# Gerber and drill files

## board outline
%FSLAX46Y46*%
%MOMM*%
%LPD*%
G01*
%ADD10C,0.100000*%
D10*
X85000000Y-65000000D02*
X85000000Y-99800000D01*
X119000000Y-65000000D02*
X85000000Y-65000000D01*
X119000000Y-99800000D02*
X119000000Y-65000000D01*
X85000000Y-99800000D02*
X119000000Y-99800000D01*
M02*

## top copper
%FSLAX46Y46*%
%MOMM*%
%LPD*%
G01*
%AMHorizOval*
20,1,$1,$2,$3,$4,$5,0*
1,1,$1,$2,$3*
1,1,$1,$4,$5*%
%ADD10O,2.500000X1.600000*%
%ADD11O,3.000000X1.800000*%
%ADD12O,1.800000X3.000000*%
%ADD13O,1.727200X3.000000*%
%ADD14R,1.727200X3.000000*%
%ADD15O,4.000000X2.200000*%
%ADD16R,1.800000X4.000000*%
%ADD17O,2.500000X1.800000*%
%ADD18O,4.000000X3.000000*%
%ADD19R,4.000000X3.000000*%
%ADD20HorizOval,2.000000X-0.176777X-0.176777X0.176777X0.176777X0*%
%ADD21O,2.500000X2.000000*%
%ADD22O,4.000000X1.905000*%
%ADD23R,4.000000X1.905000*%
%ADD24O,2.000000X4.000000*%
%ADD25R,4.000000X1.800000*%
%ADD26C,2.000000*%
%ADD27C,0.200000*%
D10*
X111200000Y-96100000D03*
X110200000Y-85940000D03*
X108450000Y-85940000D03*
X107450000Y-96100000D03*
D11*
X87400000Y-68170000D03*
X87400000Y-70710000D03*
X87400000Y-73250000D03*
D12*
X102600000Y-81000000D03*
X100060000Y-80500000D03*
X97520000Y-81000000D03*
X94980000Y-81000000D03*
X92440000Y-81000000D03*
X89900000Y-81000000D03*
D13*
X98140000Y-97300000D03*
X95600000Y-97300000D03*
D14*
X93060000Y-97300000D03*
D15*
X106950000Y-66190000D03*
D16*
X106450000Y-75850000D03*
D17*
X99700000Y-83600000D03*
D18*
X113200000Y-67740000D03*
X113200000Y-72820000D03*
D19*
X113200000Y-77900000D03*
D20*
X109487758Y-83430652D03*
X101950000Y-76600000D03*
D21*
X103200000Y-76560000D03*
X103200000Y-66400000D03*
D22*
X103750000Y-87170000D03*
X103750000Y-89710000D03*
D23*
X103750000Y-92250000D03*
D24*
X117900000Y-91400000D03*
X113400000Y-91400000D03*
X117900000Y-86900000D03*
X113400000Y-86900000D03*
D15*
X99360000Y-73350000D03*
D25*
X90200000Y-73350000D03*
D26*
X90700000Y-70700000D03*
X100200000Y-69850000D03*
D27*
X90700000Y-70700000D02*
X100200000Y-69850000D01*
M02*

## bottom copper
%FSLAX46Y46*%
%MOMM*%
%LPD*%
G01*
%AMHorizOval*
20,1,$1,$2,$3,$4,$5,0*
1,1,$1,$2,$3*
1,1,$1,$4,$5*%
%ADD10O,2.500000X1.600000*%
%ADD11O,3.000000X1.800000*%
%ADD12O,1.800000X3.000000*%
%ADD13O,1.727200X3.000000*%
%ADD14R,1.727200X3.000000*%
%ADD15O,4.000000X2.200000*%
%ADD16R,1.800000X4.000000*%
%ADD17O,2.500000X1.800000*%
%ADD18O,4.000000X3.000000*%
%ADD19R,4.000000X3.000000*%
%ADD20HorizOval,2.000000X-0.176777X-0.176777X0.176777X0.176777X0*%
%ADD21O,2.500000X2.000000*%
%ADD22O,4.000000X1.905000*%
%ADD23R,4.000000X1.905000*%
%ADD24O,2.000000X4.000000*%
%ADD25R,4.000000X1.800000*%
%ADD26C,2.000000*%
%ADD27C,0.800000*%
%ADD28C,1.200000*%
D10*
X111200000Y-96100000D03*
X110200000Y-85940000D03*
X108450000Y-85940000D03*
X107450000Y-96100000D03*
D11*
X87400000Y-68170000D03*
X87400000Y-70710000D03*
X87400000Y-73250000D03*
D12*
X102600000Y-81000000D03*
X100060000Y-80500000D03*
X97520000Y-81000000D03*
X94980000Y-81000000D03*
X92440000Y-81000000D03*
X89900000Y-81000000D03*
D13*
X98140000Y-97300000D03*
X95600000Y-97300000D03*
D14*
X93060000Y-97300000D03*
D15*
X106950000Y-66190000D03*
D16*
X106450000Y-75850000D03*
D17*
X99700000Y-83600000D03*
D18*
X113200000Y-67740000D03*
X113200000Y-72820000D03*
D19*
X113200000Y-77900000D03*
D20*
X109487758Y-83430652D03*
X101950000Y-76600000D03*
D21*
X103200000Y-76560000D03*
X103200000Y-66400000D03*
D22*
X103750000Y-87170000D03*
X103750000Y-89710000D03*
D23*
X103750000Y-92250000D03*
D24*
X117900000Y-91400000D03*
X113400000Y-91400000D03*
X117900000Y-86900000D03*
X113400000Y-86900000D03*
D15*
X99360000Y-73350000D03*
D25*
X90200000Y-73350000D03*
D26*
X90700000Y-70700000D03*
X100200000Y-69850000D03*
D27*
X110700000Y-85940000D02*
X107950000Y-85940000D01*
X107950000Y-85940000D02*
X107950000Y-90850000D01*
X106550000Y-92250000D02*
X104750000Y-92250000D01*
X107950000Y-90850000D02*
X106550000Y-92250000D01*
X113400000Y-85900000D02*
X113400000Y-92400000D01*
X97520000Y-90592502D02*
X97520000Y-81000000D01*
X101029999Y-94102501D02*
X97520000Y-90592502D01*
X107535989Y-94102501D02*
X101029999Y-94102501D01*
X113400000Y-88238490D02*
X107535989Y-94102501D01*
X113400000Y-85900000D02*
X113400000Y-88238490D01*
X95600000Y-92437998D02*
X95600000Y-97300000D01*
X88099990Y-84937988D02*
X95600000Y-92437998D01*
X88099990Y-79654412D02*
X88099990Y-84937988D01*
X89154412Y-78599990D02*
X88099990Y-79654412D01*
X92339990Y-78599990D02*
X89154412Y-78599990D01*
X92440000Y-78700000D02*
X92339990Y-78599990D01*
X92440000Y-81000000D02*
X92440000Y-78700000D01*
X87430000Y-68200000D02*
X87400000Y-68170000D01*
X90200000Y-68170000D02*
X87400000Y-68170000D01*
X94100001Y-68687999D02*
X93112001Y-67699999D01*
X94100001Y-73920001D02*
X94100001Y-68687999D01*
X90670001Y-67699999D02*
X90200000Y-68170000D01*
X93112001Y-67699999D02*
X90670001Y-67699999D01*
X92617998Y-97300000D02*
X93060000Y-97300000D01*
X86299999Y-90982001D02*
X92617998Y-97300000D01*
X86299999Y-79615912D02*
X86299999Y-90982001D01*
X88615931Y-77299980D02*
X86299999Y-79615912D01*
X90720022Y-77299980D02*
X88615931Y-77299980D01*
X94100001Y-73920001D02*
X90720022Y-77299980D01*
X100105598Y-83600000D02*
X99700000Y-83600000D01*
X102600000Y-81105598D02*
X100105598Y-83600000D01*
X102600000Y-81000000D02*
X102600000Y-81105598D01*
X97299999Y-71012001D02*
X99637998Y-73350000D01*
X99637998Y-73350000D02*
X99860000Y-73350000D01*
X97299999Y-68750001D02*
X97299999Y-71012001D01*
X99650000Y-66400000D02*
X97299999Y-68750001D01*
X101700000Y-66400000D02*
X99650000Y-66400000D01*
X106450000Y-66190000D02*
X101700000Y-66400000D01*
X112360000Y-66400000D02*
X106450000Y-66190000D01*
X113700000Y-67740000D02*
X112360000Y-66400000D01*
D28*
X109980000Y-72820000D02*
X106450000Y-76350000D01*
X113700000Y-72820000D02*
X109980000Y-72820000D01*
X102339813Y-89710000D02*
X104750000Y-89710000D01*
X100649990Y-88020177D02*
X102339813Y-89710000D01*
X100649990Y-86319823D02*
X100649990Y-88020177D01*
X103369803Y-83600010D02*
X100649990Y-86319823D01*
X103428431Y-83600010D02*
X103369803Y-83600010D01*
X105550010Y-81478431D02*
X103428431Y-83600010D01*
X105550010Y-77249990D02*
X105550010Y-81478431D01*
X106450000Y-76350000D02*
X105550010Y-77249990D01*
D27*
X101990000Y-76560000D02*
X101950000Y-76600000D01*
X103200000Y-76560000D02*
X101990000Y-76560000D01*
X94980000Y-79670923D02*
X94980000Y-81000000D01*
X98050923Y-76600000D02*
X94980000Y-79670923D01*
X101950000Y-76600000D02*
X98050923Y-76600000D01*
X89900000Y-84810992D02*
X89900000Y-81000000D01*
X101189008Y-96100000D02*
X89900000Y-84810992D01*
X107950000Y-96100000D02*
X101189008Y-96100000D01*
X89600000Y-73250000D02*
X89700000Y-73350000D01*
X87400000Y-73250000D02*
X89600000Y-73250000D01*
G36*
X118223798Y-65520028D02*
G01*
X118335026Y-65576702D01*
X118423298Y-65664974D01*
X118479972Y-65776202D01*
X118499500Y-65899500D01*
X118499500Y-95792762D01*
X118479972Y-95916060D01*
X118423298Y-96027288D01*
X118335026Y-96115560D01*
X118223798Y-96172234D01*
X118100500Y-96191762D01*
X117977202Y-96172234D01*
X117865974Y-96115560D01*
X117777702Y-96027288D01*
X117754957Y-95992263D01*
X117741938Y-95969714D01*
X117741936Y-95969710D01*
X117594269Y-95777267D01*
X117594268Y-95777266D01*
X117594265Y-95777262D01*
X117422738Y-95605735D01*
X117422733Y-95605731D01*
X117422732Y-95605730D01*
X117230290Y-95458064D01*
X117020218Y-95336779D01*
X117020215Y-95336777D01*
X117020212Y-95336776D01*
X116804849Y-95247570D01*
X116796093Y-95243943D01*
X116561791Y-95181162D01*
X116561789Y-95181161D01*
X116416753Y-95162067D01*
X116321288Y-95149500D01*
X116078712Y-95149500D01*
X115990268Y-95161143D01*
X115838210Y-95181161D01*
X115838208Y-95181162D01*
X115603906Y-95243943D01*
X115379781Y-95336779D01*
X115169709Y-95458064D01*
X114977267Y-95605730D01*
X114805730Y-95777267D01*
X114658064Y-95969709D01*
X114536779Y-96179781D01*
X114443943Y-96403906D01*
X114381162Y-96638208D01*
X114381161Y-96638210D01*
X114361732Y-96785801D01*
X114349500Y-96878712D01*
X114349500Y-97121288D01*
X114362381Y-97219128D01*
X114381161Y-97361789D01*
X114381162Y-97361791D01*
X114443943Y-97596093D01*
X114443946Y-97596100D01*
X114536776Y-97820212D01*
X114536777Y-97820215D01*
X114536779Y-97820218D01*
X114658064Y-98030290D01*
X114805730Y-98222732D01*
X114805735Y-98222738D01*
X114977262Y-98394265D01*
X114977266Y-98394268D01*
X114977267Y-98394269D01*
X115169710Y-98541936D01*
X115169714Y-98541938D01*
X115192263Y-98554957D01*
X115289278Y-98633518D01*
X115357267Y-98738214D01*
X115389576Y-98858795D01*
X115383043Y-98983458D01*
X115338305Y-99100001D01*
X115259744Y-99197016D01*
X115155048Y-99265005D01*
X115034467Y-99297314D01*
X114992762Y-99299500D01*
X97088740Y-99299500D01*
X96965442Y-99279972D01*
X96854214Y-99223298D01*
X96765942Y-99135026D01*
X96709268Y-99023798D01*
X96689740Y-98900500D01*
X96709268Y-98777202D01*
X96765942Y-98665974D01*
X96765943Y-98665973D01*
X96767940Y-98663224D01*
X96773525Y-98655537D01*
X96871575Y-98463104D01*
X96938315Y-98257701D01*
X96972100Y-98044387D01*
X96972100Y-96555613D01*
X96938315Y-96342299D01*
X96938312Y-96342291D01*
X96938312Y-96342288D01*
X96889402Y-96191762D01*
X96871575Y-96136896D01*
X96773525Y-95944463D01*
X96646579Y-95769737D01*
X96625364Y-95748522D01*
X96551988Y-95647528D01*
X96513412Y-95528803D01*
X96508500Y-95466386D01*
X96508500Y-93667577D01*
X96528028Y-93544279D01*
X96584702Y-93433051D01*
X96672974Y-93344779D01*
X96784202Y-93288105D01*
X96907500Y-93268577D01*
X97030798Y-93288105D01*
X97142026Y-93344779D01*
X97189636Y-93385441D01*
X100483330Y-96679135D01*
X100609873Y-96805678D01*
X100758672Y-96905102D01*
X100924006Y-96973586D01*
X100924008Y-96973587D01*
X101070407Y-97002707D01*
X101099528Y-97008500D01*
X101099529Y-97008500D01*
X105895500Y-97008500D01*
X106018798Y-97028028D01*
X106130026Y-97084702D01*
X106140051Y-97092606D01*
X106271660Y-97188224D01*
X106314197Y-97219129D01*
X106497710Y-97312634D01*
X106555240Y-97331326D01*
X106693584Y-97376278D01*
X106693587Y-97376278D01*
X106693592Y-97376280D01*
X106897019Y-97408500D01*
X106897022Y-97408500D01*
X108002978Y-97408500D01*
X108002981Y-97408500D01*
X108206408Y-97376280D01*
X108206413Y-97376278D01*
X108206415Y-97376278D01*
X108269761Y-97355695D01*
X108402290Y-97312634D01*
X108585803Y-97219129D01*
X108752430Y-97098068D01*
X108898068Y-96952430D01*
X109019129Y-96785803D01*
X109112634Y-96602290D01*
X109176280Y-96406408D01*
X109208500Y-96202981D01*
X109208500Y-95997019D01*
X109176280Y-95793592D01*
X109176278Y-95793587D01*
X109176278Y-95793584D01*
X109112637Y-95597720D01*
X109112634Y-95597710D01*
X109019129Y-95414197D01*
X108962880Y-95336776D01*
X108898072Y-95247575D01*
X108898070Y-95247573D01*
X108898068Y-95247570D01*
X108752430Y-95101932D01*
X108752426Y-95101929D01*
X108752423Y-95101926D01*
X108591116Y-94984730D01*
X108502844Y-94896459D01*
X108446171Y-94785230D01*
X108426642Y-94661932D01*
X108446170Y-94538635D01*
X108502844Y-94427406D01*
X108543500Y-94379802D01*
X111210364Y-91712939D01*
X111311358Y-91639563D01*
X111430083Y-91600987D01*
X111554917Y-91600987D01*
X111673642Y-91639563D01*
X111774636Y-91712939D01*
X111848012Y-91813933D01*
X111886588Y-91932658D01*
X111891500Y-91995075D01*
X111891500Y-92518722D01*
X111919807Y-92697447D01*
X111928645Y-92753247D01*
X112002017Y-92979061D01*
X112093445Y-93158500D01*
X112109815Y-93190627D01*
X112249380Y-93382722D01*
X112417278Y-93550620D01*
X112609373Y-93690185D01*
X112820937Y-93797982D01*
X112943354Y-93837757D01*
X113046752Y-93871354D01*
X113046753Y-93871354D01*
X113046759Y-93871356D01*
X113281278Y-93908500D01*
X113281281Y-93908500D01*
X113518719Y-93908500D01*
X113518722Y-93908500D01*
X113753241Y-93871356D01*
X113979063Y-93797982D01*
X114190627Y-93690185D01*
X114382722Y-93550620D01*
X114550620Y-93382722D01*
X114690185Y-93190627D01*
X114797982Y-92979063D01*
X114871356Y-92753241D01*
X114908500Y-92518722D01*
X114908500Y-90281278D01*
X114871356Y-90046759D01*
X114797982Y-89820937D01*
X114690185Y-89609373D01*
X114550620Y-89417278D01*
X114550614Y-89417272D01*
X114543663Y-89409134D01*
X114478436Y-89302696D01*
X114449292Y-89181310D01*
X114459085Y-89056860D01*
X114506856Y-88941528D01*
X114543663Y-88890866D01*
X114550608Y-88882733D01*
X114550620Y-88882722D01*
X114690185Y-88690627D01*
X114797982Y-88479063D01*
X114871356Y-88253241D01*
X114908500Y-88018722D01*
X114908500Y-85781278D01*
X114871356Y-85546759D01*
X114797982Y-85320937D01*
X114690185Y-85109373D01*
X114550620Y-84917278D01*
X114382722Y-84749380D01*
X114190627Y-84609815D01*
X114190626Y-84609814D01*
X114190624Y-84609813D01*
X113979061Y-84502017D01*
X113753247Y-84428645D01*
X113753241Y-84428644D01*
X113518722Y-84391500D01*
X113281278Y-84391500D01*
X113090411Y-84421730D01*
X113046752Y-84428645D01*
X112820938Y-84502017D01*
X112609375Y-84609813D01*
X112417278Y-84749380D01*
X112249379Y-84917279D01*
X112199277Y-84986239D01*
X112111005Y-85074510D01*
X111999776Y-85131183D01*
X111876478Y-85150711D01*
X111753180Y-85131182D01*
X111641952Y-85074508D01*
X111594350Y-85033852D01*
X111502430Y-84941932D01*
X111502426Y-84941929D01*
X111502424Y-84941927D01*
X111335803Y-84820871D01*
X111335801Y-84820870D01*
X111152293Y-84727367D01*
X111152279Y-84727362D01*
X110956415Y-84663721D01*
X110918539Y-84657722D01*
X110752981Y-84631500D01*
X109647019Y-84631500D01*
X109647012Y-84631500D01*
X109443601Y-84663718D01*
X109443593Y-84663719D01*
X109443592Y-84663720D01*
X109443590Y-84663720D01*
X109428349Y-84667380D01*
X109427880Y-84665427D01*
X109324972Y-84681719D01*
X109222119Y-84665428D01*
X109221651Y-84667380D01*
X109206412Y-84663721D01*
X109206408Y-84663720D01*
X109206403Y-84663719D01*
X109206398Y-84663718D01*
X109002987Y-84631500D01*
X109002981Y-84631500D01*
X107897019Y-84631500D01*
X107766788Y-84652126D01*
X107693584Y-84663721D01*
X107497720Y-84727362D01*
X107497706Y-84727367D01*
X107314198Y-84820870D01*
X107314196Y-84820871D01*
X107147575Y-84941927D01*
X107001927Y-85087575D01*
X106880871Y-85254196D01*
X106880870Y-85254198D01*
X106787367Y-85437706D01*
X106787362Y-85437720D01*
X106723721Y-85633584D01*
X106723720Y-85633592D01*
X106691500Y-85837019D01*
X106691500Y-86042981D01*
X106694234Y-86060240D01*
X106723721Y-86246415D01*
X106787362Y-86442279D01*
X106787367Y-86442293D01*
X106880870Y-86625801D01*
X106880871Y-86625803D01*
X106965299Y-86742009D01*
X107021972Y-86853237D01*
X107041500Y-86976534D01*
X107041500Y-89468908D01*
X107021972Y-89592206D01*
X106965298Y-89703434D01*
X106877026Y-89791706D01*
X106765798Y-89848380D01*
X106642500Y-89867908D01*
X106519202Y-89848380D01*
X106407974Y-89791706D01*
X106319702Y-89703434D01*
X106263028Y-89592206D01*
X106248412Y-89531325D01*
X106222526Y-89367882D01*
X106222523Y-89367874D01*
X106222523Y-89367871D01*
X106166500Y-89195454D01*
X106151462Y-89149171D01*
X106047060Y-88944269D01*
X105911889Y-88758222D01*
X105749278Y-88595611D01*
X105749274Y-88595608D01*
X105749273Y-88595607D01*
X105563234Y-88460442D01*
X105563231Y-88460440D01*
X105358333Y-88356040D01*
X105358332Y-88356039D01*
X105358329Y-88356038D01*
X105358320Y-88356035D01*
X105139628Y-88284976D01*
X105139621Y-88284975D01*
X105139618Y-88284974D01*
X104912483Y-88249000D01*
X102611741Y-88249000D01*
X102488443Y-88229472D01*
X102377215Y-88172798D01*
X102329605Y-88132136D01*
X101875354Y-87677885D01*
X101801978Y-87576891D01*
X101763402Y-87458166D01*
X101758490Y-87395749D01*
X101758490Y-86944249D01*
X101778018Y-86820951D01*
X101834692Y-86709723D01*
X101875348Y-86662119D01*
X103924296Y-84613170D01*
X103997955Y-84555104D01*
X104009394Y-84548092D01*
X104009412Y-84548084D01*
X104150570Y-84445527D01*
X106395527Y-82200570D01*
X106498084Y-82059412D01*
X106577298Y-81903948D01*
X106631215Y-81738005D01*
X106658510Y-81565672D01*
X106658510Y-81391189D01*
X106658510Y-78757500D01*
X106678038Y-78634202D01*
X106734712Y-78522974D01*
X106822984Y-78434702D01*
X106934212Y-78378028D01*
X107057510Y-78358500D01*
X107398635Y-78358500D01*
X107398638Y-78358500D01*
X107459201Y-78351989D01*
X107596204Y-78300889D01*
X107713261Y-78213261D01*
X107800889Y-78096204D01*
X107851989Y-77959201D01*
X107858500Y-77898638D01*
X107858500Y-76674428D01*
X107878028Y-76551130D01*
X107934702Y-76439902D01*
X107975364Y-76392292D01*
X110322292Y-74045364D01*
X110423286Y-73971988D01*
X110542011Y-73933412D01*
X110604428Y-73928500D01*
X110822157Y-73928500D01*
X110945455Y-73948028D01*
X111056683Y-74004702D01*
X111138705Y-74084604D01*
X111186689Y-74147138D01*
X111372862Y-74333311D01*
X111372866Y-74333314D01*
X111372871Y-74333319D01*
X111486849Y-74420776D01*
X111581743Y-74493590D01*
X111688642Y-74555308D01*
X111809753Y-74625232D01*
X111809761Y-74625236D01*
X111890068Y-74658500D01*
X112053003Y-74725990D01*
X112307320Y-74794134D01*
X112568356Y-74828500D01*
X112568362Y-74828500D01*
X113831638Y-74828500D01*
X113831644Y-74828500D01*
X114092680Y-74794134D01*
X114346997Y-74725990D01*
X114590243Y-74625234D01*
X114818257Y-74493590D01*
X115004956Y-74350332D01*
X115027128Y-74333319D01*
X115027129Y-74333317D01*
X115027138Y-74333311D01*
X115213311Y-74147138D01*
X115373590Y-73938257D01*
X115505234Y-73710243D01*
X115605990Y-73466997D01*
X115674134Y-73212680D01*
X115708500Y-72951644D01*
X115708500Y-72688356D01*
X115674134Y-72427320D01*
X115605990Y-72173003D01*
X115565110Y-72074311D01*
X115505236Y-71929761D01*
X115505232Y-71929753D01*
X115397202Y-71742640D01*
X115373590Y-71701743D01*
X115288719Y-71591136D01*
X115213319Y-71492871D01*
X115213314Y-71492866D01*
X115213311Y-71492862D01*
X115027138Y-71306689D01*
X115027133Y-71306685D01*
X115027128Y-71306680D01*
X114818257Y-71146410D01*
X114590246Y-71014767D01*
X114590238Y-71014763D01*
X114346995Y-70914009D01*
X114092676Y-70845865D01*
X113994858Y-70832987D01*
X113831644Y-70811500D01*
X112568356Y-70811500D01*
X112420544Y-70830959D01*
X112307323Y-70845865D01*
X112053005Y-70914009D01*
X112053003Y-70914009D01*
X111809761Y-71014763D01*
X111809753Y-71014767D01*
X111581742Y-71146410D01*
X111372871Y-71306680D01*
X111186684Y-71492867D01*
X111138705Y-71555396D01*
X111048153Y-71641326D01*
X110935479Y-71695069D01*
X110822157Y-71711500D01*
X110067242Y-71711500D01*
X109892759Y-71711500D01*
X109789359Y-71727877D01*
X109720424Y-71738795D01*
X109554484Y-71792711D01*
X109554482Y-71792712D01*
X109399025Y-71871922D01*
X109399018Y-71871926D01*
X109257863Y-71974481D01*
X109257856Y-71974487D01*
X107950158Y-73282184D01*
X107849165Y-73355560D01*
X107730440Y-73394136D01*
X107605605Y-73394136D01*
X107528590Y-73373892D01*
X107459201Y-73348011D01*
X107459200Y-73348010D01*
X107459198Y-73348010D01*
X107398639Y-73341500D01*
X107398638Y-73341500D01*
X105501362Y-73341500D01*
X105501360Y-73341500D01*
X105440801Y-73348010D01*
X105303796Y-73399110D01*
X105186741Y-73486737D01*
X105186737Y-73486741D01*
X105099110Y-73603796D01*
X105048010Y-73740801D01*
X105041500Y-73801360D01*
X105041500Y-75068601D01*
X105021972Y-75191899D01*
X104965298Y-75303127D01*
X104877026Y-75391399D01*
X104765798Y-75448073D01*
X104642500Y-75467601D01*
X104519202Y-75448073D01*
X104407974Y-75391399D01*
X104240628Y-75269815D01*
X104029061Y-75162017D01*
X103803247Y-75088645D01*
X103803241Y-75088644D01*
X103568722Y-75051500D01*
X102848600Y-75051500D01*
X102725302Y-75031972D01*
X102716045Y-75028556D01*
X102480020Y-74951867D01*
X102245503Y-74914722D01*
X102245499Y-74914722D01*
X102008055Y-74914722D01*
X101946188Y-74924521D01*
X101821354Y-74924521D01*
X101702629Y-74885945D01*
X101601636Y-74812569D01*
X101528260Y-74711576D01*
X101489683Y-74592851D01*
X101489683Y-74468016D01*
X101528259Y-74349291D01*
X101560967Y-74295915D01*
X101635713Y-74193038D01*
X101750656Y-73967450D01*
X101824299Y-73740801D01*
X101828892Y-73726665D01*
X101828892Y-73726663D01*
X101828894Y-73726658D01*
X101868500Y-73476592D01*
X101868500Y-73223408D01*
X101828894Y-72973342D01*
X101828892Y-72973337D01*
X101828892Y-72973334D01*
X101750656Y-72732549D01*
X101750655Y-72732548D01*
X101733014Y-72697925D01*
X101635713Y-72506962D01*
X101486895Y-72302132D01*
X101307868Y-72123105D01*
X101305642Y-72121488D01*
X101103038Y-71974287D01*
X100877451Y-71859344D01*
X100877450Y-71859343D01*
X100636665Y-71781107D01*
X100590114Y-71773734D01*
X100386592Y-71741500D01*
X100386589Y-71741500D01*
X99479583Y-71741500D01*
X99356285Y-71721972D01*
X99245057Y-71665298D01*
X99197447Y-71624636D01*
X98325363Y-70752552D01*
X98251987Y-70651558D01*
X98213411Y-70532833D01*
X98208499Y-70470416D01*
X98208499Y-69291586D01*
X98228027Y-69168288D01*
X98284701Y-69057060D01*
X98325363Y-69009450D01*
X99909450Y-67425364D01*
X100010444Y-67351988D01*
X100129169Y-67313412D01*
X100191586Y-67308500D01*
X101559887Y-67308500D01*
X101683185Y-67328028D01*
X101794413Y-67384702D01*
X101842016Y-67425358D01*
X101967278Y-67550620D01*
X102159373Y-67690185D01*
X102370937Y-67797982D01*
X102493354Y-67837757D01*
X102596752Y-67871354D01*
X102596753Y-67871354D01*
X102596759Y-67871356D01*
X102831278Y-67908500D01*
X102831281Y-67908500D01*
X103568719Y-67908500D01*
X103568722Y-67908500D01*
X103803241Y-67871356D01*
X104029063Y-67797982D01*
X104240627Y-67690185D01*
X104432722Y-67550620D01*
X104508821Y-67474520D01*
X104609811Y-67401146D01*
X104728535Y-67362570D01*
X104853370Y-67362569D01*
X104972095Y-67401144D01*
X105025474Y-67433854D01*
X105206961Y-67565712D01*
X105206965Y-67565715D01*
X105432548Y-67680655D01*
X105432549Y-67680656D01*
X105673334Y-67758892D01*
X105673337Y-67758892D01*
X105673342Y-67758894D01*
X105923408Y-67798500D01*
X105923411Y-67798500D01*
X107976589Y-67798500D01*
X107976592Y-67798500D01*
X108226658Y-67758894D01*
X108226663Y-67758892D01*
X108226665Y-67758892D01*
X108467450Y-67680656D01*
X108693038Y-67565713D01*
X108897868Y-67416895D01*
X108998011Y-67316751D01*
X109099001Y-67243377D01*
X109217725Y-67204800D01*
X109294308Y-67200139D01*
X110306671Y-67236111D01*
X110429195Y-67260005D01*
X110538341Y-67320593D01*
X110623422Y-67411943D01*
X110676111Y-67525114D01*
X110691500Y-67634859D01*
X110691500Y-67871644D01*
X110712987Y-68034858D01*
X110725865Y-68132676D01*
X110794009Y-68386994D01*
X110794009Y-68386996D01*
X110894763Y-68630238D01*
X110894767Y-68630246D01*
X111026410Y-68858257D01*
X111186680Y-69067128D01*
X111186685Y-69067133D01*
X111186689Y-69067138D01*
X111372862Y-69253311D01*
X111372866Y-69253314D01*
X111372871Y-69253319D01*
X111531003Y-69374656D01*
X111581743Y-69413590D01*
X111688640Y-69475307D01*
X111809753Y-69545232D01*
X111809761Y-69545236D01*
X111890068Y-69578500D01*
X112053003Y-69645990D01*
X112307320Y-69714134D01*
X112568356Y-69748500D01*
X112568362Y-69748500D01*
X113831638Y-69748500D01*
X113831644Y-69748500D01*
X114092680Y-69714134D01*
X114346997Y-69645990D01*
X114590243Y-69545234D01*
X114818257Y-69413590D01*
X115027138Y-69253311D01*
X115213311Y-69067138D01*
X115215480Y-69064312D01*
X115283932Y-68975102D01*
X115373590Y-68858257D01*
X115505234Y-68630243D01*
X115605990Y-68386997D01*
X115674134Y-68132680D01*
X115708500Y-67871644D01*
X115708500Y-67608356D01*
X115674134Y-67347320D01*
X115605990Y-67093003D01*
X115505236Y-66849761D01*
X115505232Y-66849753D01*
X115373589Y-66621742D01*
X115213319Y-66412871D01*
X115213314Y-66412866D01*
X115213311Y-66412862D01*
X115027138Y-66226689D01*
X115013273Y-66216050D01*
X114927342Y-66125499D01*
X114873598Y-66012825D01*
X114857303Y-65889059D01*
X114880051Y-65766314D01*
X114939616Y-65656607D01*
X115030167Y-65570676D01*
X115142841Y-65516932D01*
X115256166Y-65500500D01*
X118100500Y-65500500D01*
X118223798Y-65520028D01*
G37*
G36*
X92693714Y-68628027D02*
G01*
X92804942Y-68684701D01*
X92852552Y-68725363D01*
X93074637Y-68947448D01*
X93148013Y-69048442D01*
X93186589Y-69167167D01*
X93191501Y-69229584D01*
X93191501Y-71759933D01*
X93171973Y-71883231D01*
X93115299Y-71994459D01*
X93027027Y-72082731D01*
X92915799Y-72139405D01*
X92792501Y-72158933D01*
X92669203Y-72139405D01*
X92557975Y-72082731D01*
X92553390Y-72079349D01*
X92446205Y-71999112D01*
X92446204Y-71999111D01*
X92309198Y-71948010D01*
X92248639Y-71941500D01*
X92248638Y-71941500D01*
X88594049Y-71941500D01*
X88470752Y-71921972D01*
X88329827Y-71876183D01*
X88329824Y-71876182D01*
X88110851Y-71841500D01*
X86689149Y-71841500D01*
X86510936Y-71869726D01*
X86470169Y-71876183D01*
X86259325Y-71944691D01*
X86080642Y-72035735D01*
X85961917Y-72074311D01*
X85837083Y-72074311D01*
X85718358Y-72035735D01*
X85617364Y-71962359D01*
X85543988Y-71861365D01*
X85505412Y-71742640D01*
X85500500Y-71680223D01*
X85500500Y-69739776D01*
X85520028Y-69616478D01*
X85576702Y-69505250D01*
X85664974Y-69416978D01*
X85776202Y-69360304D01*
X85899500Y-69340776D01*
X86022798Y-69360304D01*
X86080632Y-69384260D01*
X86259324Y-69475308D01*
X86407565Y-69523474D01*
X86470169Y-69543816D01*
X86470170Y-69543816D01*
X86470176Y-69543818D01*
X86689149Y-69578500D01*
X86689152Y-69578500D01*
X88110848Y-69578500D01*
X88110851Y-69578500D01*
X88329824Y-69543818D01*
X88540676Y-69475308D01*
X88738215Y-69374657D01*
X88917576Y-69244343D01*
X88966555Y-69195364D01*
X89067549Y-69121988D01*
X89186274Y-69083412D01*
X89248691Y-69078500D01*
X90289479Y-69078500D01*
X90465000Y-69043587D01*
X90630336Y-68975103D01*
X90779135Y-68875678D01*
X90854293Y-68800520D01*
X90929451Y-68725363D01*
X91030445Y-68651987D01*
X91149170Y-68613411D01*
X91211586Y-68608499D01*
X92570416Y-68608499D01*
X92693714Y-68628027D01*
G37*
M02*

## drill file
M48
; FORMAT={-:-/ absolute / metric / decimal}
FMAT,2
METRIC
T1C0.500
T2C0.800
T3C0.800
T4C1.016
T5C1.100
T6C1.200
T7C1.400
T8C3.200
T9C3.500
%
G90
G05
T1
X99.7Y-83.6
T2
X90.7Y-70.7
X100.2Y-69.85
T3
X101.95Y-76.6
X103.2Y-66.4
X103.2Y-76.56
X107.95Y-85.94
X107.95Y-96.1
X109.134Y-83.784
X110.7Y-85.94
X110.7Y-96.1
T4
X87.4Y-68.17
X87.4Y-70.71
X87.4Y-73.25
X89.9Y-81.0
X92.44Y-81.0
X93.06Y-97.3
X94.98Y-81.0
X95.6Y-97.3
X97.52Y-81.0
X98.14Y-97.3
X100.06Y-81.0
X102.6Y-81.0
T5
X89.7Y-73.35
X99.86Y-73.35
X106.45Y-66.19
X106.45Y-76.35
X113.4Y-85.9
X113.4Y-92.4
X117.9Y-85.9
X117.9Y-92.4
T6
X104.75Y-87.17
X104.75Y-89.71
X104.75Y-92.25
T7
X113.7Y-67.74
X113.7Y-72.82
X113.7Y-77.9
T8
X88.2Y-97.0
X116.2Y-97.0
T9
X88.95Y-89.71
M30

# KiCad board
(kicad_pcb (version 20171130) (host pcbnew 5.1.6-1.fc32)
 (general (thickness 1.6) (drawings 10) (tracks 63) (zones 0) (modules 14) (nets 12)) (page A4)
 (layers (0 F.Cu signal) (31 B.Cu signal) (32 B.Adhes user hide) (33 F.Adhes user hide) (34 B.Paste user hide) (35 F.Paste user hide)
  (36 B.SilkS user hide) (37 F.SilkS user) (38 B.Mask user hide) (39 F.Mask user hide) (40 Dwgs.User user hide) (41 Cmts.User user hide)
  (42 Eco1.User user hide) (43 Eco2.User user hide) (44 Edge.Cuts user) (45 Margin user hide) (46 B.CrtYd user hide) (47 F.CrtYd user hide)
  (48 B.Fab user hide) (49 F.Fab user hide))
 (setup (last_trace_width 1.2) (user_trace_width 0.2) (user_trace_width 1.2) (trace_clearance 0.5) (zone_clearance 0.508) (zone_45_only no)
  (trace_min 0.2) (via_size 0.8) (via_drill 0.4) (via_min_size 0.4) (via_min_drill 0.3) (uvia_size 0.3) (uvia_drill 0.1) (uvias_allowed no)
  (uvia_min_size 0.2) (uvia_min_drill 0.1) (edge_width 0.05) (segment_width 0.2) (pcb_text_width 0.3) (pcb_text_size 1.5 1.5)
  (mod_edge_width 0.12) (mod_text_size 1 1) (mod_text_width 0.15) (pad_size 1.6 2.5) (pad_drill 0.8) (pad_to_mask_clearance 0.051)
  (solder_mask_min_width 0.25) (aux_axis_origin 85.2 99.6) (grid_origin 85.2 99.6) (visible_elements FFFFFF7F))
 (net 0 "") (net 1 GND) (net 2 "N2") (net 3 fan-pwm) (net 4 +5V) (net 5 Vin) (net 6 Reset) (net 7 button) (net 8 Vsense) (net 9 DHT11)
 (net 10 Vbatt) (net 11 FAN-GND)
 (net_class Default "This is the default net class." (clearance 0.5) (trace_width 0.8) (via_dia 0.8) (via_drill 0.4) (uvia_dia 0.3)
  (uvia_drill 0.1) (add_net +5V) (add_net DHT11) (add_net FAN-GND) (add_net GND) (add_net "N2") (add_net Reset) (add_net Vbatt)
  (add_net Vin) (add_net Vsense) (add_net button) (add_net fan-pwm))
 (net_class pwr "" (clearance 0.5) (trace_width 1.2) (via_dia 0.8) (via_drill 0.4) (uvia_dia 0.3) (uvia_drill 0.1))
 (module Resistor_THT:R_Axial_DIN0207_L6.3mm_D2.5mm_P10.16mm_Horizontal (layer F.Cu) (at 110.7 85.94 270)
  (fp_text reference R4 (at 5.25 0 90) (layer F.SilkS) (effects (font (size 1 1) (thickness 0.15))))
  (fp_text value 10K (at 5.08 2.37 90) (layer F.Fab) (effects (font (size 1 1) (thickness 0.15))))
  (pad 2 thru_hole oval (at 10.16 0 270) (size 1.6 2.5) (drill 0.8 (offset 0 -0.5)) (layers *.Cu *.Mask) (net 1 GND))
  (pad 1 thru_hole oval (at 0 0 270) (size 1.6 2.5) (drill 0.8 (offset 0 0.5)) (layers *.Cu *.Mask) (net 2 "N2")))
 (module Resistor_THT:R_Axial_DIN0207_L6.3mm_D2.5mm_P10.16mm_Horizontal (layer F.Cu) (at 107.95 96.1 90)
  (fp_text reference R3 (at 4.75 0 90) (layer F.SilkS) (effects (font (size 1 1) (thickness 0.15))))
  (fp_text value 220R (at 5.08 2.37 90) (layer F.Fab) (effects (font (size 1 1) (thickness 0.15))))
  (pad 2 thru_hole oval (at 10.16 0 90) (size 1.6 2.5) (drill 0.8 (offset 0 0.5)) (layers *.Cu *.Mask) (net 2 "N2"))
  (pad 1 thru_hole oval (at 0 0 90) (size 1.6 2.5) (drill 0.8 (offset 0 -0.5)) (layers *.Cu *.Mask) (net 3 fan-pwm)))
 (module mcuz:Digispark (layer F.Cu) (at 96.25 81)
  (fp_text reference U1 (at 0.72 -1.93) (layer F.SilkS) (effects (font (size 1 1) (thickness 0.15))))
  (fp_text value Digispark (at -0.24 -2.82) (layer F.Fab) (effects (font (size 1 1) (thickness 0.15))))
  (pad 9 thru_hole oval (at -8.85 -12.83) (size 3 1.8) (drill 1.016) (layers *.Cu *.Mask) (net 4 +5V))
  (pad 8 thru_hole oval (at -8.85 -10.29) (size 3 1.8) (drill 1.016) (layers *.Cu *.Mask) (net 1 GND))
  (pad 7 thru_hole oval (at -8.85 -7.75) (size 3 1.8) (drill 1.016) (layers *.Cu *.Mask) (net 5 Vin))
  (pad 6 thru_hole oval (at 6.35 0) (size 1.8 3) (drill 1.016) (layers *.Cu *.Mask) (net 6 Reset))
  (pad 5 thru_hole oval (at 3.81 0) (size 1.8 3) (drill 1.016 (offset 0 -0.5)) (layers *.Cu *.Mask))
  (pad 4 thru_hole oval (at 1.27 0) (size 1.8 3) (drill 1.016) (layers *.Cu *.Mask) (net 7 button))
  (pad 3 thru_hole oval (at -1.27 0) (size 1.8 3) (drill 1.016) (layers *.Cu *.Mask) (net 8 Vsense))
  (pad 2 thru_hole oval (at -3.81 0) (size 1.8 3) (drill 1.016) (layers *.Cu *.Mask) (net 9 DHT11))
  (pad 1 thru_hole oval (at -6.35 0) (size 1.8 3) (drill 1.016) (layers *.Cu *.Mask) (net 3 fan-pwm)))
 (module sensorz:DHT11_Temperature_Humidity (layer F.Cu) (at 95.6 97.3)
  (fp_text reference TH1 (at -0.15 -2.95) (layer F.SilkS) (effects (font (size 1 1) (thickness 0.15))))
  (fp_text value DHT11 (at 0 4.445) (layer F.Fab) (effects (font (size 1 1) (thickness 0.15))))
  (pad 3 thru_hole oval (at 2.54 0 90) (size 3 1.7272) (drill 1.016) (layers *.Cu *.Mask) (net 1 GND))
  (pad 2 thru_hole oval (at 0 0 90) (size 3 1.7272) (drill 1.016) (layers *.Cu *.Mask) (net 9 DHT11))
  (pad 1 thru_hole rect (at -2.54 0 90) (size 3 1.7272) (drill 1.016) (layers *.Cu *.Mask) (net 4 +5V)))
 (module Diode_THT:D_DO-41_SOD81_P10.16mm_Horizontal (layer F.Cu) (at 106.45 76.35 90)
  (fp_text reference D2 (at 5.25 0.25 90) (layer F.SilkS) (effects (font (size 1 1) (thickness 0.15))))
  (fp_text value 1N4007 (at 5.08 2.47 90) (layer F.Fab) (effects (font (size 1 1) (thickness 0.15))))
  (pad 2 thru_hole oval (at 10.16 0 180) (size 4 2.2) (drill 1.1 (offset -0.5 0)) (layers *.Cu *.Mask) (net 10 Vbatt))
  (pad 1 thru_hole rect (at 0 0 90) (size 4 1.8) (drill 1.1 (offset 0.5 0)) (layers *.Cu *.Mask) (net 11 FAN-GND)))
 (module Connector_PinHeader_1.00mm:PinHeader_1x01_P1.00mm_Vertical (layer F.Cu) (at 99.7 83.6)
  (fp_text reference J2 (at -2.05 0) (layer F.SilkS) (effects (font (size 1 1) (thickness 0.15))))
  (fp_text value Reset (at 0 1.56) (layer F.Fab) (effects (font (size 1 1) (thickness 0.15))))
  (pad 1 thru_hole oval (at 0 0) (size 2.5 1.8) (drill 0.5) (layers *.Cu *.Mask) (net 6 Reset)))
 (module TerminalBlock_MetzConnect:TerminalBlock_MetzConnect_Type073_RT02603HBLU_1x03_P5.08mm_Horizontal (layer F.Cu) (at 113.7 77.9 90)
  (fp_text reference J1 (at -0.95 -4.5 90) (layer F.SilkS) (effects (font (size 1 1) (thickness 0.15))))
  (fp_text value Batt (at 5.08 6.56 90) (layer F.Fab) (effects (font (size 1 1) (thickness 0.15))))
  (pad 3 thru_hole oval (at 10.16 0 90) (size 3 4) (drill 1.4 (offset 0 -0.5)) (layers *.Cu *.Mask) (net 10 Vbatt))
  (pad 2 thru_hole oval (at 5.08 0 90) (size 3 4) (drill 1.4 (offset 0 -0.5)) (layers *.Cu *.Mask) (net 11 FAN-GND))
  (pad 1 thru_hole rect (at 0 0 90) (size 3 4) (drill 1.4 (offset 0 -0.5)) (layers *.Cu *.Mask) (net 1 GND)))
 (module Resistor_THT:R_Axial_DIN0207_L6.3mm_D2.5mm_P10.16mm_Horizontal (layer F.Cu) (at 101.95 76.6 315)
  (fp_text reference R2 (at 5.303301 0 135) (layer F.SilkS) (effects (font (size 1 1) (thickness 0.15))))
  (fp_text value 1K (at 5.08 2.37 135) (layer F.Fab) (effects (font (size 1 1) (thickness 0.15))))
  (pad 2 thru_hole oval (at 10.16 0 315) (size 2 2.5) (drill 0.8 (offset 0 -0.5)) (layers *.Cu *.Mask) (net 1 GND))
  (pad 1 thru_hole oval (at 0 0 315) (size 2 2.5) (drill 0.8) (layers *.Cu *.Mask) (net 8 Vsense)))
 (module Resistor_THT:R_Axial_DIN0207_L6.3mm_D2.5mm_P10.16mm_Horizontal (layer F.Cu) (at 103.2 66.4 270)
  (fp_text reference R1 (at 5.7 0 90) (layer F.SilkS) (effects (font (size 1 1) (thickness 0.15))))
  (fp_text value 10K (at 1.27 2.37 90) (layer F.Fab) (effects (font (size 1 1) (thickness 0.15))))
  (pad 2 thru_hole oval (at 10.16 0 270) (size 2 2.5) (drill 0.8) (layers *.Cu *.Mask) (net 8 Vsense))
  (pad 1 thru_hole oval (at 0 0 270) (size 2 2.5) (drill 0.8) (layers *.Cu *.Mask) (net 10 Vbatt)))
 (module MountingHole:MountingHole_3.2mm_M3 (layer F.Cu) (at 116.2 97)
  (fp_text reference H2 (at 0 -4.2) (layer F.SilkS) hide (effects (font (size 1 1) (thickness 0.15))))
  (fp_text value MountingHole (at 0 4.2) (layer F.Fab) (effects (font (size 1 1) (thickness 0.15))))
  (pad 1 np_thru_hole circle (at 0 0) (size 3.2 3.2) (drill 3.2) (layers *.Cu *.Mask)))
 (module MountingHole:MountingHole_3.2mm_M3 (layer F.Cu) (at 88.2 97)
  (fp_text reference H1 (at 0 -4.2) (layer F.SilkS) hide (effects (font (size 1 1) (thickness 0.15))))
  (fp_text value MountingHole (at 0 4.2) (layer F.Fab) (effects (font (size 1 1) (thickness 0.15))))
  (pad 1 np_thru_hole circle (at 0 0) (size 3.2 3.2) (drill 3.2) (layers *.Cu *.Mask)))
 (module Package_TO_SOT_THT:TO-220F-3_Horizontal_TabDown (layer F.Cu) (at 104.75 92.25 90)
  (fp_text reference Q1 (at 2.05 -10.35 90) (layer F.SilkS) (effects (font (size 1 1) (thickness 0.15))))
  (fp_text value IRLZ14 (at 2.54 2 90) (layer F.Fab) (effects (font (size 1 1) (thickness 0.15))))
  (pad 3 thru_hole oval (at 5.08 0 90) (size 1.905 4) (drill 1.2 (offset 0 -1)) (layers *.Cu *.Mask) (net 1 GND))
  (pad 2 thru_hole oval (at 2.54 0 90) (size 1.905 4) (drill 1.2 (offset 0 -1)) (layers *.Cu *.Mask) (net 11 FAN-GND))
  (pad 1 thru_hole rect (at 0 0 90) (size 1.905 4) (drill 1.2 (offset 0 -1)) (layers *.Cu *.Mask) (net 2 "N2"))
  (pad "" np_thru_hole oval (at 2.54 -15.8 90) (size 3.5 3.5) (drill 3.5) (layers *.Cu *.Mask)))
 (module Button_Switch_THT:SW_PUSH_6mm (layer F.Cu) (at 117.9 85.9 270)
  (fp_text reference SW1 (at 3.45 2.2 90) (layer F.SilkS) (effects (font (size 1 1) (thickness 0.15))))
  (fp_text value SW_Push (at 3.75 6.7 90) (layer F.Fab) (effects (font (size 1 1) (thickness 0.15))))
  (pad 1 thru_hole oval (at 6.5 0 270) (size 4 2) (drill 1.1 (offset -1 0)) (layers *.Cu *.Mask) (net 1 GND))
  (pad 2 thru_hole oval (at 6.5 4.5) (size 2 4) (drill 1.1 (offset 0 -1)) (layers *.Cu *.Mask) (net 7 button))
  (pad 1 thru_hole oval (at 0 0) (size 2 4) (drill 1.1 (offset 0 1)) (layers *.Cu *.Mask) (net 1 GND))
  (pad 2 thru_hole oval (at 0 4.5) (size 2 4) (drill 1.1 (offset 0 1)) (layers *.Cu *.Mask) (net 7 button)))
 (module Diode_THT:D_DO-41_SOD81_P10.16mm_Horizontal (layer F.Cu) (at 89.7 73.35)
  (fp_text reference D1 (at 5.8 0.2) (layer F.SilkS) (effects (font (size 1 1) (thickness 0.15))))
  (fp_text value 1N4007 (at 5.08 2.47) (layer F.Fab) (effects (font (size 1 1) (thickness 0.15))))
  (pad 2 thru_hole oval (at 10.16 0) (size 4 2.2) (drill 1.1 (offset -0.5 0)) (layers *.Cu *.Mask) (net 10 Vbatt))
  (pad 1 thru_hole rect (at 0 0) (size 4 1.8) (drill 1.1 (offset 0.5 0)) (layers *.Cu *.Mask) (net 5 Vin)))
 (gr_line (start 85 65) (end 85 99.8) (layer Edge.Cuts) (width 0.1))
 (gr_line (start 119 65) (end 85 65) (layer Edge.Cuts) (width 0.1))
 (gr_line (start 119 99.8) (end 119 65) (layer Edge.Cuts) (width 0.1))
 (gr_line (start 85 99.8) (end 119 99.8) (layer Edge.Cuts) (width 0.1))
 (via (at 90.7 70.7) (size 2) (drill 0.8) (layers F.Cu B.Cu) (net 1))
 (via (at 100.2 69.85) (size 2) (drill 0.8) (layers F.Cu B.Cu) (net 1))
 (segment (start 90.7 70.7) (end 100.2 69.85) (width 0.2) (layer F.Cu) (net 1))
 (segment (start 110.7 85.94) (end 107.95 85.94) (width 0.8) (layer B.Cu) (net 2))
 (segment (start 107.95 85.94) (end 107.95 90.85) (width 0.8) (layer B.Cu) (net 2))
 (segment (start 106.55 92.25) (end 104.75 92.25) (width 0.8) (layer B.Cu) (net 2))
 (segment (start 107.95 90.85) (end 106.55 92.25) (width 0.8) (layer B.Cu) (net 2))
 (segment (start 113.4 85.9) (end 113.4 92.4) (width 0.8) (layer B.Cu) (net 7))
 (segment (start 97.52 90.592502) (end 97.52 81) (width 0.8) (layer B.Cu) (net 7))
 (segment (start 101.029999 94.102501) (end 97.52 90.592502) (width 0.8) (layer B.Cu) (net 7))
 (segment (start 107.535989 94.102501) (end 101.029999 94.102501) (width 0.8) (layer B.Cu) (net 7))
 (segment (start 113.4 88.23849) (end 107.535989 94.102501) (width 0.8) (layer B.Cu) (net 7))
 (segment (start 113.4 85.9) (end 113.4 88.23849) (width 0.8) (layer B.Cu) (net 7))
 (segment (start 95.6 92.437998) (end 95.6 97.3) (width 0.8) (layer B.Cu) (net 9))
 (segment (start 88.09999 84.937988) (end 95.6 92.437998) (width 0.8) (layer B.Cu) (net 9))
 (segment (start 88.09999 79.654412) (end 88.09999 84.937988) (width 0.8) (layer B.Cu) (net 9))
 (segment (start 89.154412 78.59999) (end 88.09999 79.654412) (width 0.8) (layer B.Cu) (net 9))
 (segment (start 92.33999 78.59999) (end 89.154412 78.59999) (width 0.8) (layer B.Cu) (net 9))
 (segment (start 92.44 78.7) (end 92.33999 78.59999) (width 0.8) (layer B.Cu) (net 9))
 (segment (start 92.44 81) (end 92.44 78.7) (width 0.8) (layer B.Cu) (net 9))
 (segment (start 87.43 68.2) (end 87.4 68.17) (width 0.8) (layer B.Cu) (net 4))
 (segment (start 90.2 68.17) (end 87.4 68.17) (width 0.8) (layer B.Cu) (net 4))
 (segment (start 94.100001 68.687999) (end 93.112001 67.699999) (width 0.8) (layer B.Cu) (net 4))
 (segment (start 94.100001 73.920001) (end 94.100001 68.687999) (width 0.8) (layer B.Cu) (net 4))
 (segment (start 90.670001 67.699999) (end 90.2 68.17) (width 0.8) (layer B.Cu) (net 4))
 (segment (start 93.112001 67.699999) (end 90.670001 67.699999) (width 0.8) (layer B.Cu) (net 4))
 (segment (start 92.617998 97.3) (end 93.06 97.3) (width 0.8) (layer B.Cu) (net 4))
 (segment (start 86.299999 90.982001) (end 92.617998 97.3) (width 0.8) (layer B.Cu) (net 4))
 (segment (start 86.299999 79.615912) (end 86.299999 90.982001) (width 0.8) (layer B.Cu) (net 4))
 (segment (start 88.615931 77.29998) (end 86.299999 79.615912) (width 0.8) (layer B.Cu) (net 4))
 (segment (start 90.720022 77.29998) (end 88.615931 77.29998) (width 0.8) (layer B.Cu) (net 4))
 (segment (start 94.100001 73.920001) (end 90.720022 77.29998) (width 0.8) (layer B.Cu) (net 4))
 (segment (start 100.105598 83.6) (end 99.7 83.6) (width 0.8) (layer B.Cu) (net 6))
 (segment (start 102.6 81.105598) (end 100.105598 83.6) (width 0.8) (layer B.Cu) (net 6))
 (segment (start 102.6 81) (end 102.6 81.105598) (width 0.8) (layer B.Cu) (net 6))
 (segment (start 97.299999 71.012001) (end 99.637998 73.35) (width 0.8) (layer B.Cu) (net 10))
 (segment (start 99.637998 73.35) (end 99.86 73.35) (width 0.8) (layer B.Cu) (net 10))
 (segment (start 97.299999 68.750001) (end 97.299999 71.012001) (width 0.8) (layer B.Cu) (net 10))
 (segment (start 99.65 66.4) (end 97.299999 68.750001) (width 0.8) (layer B.Cu) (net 10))
 (segment (start 101.7 66.4) (end 99.65 66.4) (width 0.8) (layer B.Cu) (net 10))
 (segment (start 106.45 66.19) (end 101.7 66.4) (width 0.8) (layer B.Cu) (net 10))
 (segment (start 112.36 66.4) (end 106.45 66.19) (width 0.8) (layer B.Cu) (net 10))
 (segment (start 113.7 67.74) (end 112.36 66.4) (width 0.8) (layer B.Cu) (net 10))
 (segment (start 109.98 72.82) (end 106.45 76.35) (width 1.2) (layer B.Cu) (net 11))
 (segment (start 113.7 72.82) (end 109.98 72.82) (width 1.2) (layer B.Cu) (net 11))
 (segment (start 102.339813 89.71) (end 104.75 89.71) (width 1.2) (layer B.Cu) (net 11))
 (segment (start 100.64999 88.020177) (end 102.339813 89.71) (width 1.2) (layer B.Cu) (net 11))
 (segment (start 100.64999 86.319823) (end 100.64999 88.020177) (width 1.2) (layer B.Cu) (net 11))
 (segment (start 103.369803 83.60001) (end 100.64999 86.319823) (width 1.2) (layer B.Cu) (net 11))
 (segment (start 103.428431 83.60001) (end 103.369803 83.60001) (width 1.2) (layer B.Cu) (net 11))
 (segment (start 105.55001 81.478431) (end 103.428431 83.60001) (width 1.2) (layer B.Cu) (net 11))
 (segment (start 105.55001 77.24999) (end 105.55001 81.478431) (width 1.2) (layer B.Cu) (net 11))
 (segment (start 106.45 76.35) (end 105.55001 77.24999) (width 1.2) (layer B.Cu) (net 11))
 (segment (start 101.99 76.56) (end 101.95 76.6) (width 0.8) (layer B.Cu) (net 8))
 (segment (start 103.2 76.56) (end 101.99 76.56) (width 0.8) (layer B.Cu) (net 8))
 (segment (start 94.98 79.670923) (end 94.98 81) (width 0.8) (layer B.Cu) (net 8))
 (segment (start 98.050923 76.6) (end 94.98 79.670923) (width 0.8) (layer B.Cu) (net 8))
 (segment (start 101.95 76.6) (end 98.050923 76.6) (width 0.8) (layer B.Cu) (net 8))
 (segment (start 89.9 84.810992) (end 89.9 81) (width 0.8) (layer B.Cu) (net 3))
 (segment (start 101.189008 96.1) (end 89.9 84.810992) (width 0.8) (layer B.Cu) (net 3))
 (segment (start 107.95 96.1) (end 101.189008 96.1) (width 0.8) (layer B.Cu) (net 3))
 (segment (start 89.6 73.25) (end 89.7 73.35) (width 0.8) (layer B.Cu) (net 5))
 (segment (start 87.4 73.25) (end 89.6 73.25) (width 0.8) (layer B.Cu) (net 5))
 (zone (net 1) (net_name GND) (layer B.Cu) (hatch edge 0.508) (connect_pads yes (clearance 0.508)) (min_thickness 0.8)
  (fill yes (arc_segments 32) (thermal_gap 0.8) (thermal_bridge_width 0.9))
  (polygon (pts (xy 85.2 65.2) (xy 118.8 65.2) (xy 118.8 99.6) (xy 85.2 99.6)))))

